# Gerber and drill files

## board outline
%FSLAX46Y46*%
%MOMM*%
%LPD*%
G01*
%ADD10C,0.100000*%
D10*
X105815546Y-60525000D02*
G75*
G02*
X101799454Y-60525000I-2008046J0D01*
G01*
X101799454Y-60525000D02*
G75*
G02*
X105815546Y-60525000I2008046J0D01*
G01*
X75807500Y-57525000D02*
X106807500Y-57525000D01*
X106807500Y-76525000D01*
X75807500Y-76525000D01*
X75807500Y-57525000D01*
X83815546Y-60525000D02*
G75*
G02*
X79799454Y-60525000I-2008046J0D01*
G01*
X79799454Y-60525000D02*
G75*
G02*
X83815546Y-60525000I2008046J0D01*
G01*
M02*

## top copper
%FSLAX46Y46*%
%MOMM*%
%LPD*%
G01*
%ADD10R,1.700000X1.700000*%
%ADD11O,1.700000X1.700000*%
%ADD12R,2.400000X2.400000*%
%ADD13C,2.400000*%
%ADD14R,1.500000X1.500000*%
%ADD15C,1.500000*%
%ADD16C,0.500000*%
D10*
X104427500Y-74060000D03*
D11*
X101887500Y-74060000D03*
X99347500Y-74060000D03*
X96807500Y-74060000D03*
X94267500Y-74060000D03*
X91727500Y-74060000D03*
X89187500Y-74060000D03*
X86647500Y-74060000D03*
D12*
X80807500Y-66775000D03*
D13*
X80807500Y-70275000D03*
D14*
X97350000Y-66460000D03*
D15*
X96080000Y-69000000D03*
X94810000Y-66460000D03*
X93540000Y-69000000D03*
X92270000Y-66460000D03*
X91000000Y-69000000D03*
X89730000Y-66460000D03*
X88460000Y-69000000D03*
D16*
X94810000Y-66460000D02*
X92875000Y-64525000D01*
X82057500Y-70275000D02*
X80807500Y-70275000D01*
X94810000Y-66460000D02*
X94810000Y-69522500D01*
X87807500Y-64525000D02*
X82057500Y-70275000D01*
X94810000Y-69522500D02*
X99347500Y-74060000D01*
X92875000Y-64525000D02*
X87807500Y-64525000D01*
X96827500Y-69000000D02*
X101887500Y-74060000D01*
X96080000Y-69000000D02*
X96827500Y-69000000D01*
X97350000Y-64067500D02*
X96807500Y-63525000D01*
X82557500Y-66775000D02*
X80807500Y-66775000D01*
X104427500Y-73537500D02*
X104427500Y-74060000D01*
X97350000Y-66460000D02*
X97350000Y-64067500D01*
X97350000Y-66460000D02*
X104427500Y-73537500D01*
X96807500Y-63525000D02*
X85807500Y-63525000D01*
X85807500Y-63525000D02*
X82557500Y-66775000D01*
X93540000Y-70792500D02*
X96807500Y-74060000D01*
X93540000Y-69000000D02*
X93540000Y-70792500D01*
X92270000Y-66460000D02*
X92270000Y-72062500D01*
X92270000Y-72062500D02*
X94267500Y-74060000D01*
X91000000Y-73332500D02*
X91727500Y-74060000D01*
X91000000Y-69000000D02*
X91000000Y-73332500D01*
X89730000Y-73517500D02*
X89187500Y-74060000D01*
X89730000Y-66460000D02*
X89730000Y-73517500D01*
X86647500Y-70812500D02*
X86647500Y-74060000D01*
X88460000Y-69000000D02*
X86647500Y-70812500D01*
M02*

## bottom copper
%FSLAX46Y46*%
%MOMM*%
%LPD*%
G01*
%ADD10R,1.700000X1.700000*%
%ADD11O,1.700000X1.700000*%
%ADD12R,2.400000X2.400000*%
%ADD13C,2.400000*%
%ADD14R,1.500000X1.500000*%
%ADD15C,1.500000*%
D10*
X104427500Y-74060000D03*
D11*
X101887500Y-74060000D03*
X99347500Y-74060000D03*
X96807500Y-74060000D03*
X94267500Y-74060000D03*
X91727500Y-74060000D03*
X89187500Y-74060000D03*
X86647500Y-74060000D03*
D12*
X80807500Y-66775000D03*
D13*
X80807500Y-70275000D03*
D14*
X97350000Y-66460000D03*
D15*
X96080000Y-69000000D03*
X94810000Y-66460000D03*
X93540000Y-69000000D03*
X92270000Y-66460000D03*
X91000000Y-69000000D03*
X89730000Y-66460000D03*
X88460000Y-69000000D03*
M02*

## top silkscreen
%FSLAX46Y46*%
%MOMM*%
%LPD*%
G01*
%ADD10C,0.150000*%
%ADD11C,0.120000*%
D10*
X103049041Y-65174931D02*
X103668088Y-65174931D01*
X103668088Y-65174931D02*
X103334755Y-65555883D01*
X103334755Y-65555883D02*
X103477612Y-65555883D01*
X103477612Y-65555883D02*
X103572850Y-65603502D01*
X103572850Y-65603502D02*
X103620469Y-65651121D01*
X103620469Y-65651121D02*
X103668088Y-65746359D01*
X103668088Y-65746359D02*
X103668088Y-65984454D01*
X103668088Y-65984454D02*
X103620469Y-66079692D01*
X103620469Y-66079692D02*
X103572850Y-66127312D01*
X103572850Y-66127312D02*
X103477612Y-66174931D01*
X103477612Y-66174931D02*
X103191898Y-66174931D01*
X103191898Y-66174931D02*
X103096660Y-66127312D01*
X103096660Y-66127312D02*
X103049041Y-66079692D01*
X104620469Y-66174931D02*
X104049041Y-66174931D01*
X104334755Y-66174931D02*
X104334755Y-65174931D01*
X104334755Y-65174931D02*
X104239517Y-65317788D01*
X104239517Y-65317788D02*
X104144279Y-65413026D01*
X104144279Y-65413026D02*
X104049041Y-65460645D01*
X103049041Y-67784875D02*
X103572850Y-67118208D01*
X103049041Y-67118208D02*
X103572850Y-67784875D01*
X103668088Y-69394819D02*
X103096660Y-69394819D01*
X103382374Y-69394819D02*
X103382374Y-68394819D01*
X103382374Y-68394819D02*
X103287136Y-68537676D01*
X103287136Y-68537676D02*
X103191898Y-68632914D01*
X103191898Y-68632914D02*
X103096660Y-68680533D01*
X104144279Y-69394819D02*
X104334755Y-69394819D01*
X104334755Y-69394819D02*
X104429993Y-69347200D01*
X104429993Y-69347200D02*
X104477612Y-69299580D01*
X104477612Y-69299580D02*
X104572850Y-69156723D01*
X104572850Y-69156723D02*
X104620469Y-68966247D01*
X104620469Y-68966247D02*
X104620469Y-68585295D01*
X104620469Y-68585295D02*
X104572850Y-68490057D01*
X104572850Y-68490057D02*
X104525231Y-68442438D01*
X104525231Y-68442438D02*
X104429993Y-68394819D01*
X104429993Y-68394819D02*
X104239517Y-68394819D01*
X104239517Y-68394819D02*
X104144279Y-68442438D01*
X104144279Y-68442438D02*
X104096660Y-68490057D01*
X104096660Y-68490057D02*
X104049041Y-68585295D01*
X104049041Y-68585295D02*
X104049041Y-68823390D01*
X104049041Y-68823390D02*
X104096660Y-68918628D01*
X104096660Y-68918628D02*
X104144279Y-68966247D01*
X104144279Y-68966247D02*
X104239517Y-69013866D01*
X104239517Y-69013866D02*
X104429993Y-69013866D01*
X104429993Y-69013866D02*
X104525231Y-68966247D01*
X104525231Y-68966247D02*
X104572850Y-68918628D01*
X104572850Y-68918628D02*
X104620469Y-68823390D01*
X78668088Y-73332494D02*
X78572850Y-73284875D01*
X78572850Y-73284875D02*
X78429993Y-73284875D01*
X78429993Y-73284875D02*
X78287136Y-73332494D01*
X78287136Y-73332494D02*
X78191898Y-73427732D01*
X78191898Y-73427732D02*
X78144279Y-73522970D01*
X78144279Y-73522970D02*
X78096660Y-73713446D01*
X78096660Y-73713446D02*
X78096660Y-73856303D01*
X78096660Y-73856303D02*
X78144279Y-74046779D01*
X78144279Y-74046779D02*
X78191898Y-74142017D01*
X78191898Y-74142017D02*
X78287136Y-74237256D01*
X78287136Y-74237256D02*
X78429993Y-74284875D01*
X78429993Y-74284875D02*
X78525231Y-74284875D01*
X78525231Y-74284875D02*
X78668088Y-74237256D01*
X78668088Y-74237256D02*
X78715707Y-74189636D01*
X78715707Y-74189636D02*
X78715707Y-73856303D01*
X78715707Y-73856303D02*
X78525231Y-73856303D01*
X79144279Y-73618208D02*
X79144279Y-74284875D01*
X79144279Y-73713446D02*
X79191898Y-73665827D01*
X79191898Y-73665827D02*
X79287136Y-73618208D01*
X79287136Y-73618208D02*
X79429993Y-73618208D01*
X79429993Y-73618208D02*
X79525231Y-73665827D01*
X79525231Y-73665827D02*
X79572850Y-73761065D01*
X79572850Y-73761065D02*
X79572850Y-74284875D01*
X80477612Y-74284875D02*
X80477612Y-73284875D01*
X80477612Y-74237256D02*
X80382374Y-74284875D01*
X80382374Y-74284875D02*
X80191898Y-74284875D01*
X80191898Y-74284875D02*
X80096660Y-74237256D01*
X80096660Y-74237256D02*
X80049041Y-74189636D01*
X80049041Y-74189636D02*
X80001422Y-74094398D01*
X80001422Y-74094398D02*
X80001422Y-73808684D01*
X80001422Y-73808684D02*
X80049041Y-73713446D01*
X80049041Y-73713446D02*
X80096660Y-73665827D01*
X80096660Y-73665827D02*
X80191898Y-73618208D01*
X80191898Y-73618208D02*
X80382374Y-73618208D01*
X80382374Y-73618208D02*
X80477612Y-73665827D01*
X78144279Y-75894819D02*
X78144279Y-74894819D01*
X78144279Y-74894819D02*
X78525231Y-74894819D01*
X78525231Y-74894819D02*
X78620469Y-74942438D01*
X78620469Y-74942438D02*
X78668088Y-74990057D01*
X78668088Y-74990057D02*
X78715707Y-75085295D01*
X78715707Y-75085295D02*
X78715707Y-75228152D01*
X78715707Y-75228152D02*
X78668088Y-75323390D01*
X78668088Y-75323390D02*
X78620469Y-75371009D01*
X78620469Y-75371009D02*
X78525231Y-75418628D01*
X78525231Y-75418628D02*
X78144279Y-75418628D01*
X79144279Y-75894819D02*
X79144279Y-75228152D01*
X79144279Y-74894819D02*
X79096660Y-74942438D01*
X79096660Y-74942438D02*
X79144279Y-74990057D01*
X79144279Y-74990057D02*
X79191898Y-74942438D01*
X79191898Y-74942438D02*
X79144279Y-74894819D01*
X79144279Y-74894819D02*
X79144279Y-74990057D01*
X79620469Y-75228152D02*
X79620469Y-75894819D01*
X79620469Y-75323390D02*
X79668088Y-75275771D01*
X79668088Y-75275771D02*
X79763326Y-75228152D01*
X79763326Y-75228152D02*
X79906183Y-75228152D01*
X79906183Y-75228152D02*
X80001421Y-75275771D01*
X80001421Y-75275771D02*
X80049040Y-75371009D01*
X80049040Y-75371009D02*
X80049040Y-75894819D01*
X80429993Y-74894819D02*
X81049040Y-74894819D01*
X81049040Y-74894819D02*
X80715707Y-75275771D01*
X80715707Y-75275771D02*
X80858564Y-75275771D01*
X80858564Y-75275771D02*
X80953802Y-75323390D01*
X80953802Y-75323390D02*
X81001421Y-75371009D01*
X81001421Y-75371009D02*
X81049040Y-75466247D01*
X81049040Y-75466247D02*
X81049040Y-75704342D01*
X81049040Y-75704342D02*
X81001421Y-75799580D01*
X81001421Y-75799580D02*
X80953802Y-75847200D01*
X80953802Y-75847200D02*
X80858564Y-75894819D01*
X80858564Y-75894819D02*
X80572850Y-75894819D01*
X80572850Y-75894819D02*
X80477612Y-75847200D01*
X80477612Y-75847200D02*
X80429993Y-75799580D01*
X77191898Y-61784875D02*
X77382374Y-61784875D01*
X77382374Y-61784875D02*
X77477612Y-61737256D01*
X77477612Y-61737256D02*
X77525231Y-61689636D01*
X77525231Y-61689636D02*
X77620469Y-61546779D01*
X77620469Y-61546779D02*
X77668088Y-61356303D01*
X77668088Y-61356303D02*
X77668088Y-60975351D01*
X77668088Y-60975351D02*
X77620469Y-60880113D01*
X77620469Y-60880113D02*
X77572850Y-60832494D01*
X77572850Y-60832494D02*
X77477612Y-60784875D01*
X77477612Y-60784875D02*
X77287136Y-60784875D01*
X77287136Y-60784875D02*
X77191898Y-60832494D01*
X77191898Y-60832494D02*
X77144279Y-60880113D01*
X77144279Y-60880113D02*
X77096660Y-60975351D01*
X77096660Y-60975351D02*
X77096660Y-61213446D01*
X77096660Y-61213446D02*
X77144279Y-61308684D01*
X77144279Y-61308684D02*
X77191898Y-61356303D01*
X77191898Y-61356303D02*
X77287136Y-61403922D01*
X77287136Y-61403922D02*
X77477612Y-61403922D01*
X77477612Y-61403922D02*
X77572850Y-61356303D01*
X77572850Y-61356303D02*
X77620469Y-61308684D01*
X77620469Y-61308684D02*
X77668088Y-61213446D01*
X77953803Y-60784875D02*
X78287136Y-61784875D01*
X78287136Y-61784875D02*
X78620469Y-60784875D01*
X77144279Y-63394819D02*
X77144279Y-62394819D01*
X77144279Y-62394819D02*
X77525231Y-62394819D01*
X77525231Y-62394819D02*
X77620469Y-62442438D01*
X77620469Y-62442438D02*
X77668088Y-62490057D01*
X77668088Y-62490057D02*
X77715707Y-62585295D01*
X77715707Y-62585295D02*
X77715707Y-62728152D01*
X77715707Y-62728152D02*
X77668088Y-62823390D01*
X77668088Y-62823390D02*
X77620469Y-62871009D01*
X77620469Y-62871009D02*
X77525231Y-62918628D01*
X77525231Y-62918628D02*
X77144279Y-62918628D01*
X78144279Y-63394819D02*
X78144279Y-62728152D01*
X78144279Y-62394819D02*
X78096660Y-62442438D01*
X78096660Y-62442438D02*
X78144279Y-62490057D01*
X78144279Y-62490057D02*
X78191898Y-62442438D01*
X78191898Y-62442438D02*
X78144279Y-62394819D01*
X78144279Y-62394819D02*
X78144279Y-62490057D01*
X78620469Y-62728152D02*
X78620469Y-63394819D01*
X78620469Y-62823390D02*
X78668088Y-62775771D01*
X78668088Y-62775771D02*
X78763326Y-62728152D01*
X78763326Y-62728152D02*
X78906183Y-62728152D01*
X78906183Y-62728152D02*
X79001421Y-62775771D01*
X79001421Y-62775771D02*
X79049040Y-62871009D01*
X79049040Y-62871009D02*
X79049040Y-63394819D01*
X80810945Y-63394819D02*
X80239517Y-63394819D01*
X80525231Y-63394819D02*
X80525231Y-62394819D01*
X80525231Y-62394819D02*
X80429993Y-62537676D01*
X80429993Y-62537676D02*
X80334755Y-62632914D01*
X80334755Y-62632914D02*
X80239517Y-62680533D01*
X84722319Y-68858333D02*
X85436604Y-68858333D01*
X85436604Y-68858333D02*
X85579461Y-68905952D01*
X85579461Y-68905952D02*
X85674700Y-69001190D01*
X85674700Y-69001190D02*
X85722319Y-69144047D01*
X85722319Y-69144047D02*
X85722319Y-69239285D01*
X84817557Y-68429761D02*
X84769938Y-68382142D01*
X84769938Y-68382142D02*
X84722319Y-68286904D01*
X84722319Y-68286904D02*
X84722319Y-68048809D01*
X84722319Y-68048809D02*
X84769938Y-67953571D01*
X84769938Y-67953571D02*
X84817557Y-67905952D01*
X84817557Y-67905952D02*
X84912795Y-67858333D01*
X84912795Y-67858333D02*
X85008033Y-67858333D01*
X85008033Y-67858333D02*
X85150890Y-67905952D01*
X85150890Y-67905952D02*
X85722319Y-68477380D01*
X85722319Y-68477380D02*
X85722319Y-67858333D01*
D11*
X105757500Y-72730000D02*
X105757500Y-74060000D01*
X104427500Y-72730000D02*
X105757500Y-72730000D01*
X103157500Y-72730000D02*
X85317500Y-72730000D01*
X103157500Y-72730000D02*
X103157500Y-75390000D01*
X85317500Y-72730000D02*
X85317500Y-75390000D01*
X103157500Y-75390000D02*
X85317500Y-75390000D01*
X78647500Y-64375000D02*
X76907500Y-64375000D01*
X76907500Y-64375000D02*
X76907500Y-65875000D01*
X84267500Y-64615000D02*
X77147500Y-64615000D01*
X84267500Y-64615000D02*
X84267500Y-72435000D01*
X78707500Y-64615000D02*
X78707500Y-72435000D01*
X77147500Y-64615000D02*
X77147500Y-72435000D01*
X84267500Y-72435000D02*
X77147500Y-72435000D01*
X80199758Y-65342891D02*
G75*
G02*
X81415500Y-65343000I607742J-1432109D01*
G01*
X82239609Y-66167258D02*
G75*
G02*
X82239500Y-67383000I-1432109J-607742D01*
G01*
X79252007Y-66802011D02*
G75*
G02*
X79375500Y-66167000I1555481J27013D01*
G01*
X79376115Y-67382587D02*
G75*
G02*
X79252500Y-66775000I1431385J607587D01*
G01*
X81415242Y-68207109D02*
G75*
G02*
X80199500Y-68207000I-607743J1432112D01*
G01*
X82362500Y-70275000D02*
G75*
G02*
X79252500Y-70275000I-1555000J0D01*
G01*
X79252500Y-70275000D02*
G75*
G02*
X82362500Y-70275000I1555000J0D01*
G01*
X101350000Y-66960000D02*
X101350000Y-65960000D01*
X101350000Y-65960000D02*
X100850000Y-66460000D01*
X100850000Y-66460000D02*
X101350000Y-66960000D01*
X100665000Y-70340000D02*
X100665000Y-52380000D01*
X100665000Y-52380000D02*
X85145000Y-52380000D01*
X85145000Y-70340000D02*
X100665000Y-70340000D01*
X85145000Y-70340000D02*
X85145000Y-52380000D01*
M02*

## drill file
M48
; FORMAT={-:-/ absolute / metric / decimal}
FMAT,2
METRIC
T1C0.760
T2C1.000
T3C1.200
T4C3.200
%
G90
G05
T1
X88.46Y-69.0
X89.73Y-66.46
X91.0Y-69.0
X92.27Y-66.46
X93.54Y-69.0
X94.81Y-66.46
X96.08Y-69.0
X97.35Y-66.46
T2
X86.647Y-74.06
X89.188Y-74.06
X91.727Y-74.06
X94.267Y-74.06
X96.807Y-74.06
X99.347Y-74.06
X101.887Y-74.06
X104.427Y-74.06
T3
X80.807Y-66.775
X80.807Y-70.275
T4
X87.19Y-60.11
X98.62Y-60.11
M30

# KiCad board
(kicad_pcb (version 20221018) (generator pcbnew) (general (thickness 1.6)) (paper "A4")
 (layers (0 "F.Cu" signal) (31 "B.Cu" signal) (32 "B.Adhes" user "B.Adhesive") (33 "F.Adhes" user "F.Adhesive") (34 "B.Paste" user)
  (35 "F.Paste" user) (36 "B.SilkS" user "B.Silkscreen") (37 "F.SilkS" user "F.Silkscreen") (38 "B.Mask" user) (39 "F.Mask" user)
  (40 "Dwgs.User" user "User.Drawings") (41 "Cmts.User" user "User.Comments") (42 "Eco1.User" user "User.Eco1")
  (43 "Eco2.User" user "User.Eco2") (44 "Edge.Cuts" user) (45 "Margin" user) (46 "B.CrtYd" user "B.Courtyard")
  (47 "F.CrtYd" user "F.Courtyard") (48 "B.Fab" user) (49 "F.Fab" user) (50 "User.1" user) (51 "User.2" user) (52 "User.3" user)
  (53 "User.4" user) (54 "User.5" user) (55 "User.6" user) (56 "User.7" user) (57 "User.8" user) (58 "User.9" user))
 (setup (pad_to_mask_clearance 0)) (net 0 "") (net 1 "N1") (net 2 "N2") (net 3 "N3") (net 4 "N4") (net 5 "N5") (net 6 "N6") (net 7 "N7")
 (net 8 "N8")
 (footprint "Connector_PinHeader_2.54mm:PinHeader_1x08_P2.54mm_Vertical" (layer "F.Cu") (at 104.4275 74.06 -90)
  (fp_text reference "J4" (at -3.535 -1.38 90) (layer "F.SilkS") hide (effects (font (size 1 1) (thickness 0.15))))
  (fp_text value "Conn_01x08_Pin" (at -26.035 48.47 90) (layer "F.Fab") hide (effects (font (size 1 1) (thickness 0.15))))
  (fp_line (start -1.33 -1.33) (end 0 -1.33) (stroke (width 0.12) (type solid)) (layer "F.SilkS"))
  (fp_line (start -1.33 0) (end -1.33 -1.33) (stroke (width 0.12) (type solid)) (layer "F.SilkS"))
  (fp_line (start -1.33 1.27) (end -1.33 19.11) (stroke (width 0.12) (type solid)) (layer "F.SilkS"))
  (fp_line (start -1.33 1.27) (end 1.33 1.27) (stroke (width 0.12) (type solid)) (layer "F.SilkS"))
  (fp_line (start -1.33 19.11) (end 1.33 19.11) (stroke (width 0.12) (type solid)) (layer "F.SilkS"))
  (fp_line (start 1.33 1.27) (end 1.33 19.11) (stroke (width 0.12) (type solid)) (layer "F.SilkS"))
  (pad "1" thru_hole rect (at 0 0 270) (size 1.7 1.7) (drill 1) (layers "*.Cu" "*.Mask") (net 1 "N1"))
  (pad "2" thru_hole oval (at 0 2.54 270) (size 1.7 1.7) (drill 1) (layers "*.Cu" "*.Mask") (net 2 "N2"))
  (pad "3" thru_hole oval (at 0 5.08 270) (size 1.7 1.7) (drill 1) (layers "*.Cu" "*.Mask") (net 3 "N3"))
  (pad "4" thru_hole oval (at 0 7.62 270) (size 1.7 1.7) (drill 1) (layers "*.Cu" "*.Mask") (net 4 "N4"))
  (pad "5" thru_hole oval (at 0 10.16 270) (size 1.7 1.7) (drill 1) (layers "*.Cu" "*.Mask") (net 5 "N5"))
  (pad "6" thru_hole oval (at 0 12.7 270) (size 1.7 1.7) (drill 1) (layers "*.Cu" "*.Mask") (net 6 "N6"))
  (pad "7" thru_hole oval (at 0 15.24 270) (size 1.7 1.7) (drill 1) (layers "*.Cu" "*.Mask") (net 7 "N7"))
  (pad "8" thru_hole oval (at 0 17.78 270) (size 1.7 1.7) (drill 1) (layers "*.Cu" "*.Mask") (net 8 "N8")))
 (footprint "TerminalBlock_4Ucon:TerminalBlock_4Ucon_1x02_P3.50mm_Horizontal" (layer "F.Cu") (at 80.8075 66.775 -90)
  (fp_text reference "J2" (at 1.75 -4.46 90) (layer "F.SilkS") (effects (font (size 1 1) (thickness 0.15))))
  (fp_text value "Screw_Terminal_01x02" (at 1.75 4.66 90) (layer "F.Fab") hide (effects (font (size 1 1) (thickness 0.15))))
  (fp_line (start -2.4 2.16) (end -2.4 3.9) (stroke (width 0.12) (type solid)) (layer "F.SilkS"))
  (fp_line (start -2.4 3.9) (end -0.9 3.9) (stroke (width 0.12) (type solid)) (layer "F.SilkS"))
  (fp_line (start -2.16 -3.46) (end -2.16 3.66) (stroke (width 0.12) (type solid)) (layer "F.SilkS"))
  (fp_line (start -2.16 -3.46) (end 5.66 -3.46) (stroke (width 0.12) (type solid)) (layer "F.SilkS"))
  (fp_line (start -2.16 2.1) (end 5.66 2.1) (stroke (width 0.12) (type solid)) (layer "F.SilkS"))
  (fp_line (start -2.16 3.66) (end 5.66 3.66) (stroke (width 0.12) (type solid)) (layer "F.SilkS"))
  (fp_line (start 5.66 -3.46) (end 5.66 3.66) (stroke (width 0.12) (type solid)) (layer "F.SilkS"))
  (fp_arc (start -1.432109 0.607742) (mid -1.555727 -0.00014) (end -1.432 -0.608) (stroke (width 0.12) (type solid)) (layer "F.SilkS"))
  (fp_arc (start -0.607742 -1.432109) (mid 0.00014 -1.555727) (end 0.608 -1.432) (stroke (width 0.12) (type solid)) (layer "F.SilkS"))
  (fp_arc (start 0.027011 1.555493) (mid -0.296984 1.527118) (end -0.608 1.432) (stroke (width 0.12) (type solid)) (layer "F.SilkS"))
  (fp_arc (start 0.607587 1.431385) (mid 0.310017 1.523783) (end 0 1.555) (stroke (width 0.12) (type solid)) (layer "F.SilkS"))
  (fp_arc (start 1.432109 -0.607742) (mid 1.555727 0.00014) (end 1.432 0.608) (stroke (width 0.12) (type solid)) (layer "F.SilkS"))
  (fp_circle (center 3.5 0) (end 5.055 0) (stroke (width 0.12) (type solid)) (fill none) (layer "F.SilkS"))
  (pad "1" thru_hole rect (at 0 0 270) (size 2.4 2.4) (drill 1.2) (layers "*.Cu" "*.Mask") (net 1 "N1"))
  (pad "2" thru_hole circle (at 3.5 0 270) (size 2.4 2.4) (drill 1.2) (layers "*.Cu" "*.Mask") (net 3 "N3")))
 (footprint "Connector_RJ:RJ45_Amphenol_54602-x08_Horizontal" (layer "F.Cu") (at 97.35 66.46 180)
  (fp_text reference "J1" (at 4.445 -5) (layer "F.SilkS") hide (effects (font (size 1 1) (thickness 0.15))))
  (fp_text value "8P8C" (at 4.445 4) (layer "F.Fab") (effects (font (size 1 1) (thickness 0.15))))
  (fp_line (start -4 -0.5) (end -4 0.5) (stroke (width 0.12) (type solid)) (layer "F.SilkS"))
  (fp_line (start -4 0.5) (end -3.5 0) (stroke (width 0.12) (type solid)) (layer "F.SilkS"))
  (fp_line (start -3.5 0) (end -4 -0.5) (stroke (width 0.12) (type solid)) (layer "F.SilkS"))
  (fp_line (start -3.315 -3.88) (end -3.315 14.08) (stroke (width 0.12) (type solid)) (layer "F.SilkS"))
  (fp_line (start -3.315 14.08) (end 12.205 14.08) (stroke (width 0.12) (type solid)) (layer "F.SilkS"))
  (fp_line (start 12.205 -3.88) (end -3.315 -3.88) (stroke (width 0.12) (type solid)) (layer "F.SilkS"))
  (fp_line (start 12.205 -3.88) (end 12.205 14.08) (stroke (width 0.12) (type solid)) (layer "F.SilkS"))
  (pad "" np_thru_hole circle (at -1.27 6.35 180) (size 3.2 3.2) (drill 3.2) (layers "*.Cu" "*.Mask"))
  (pad "" np_thru_hole circle (at 10.16 6.35 180) (size 3.2 3.2) (drill 3.2) (layers "*.Cu" "*.Mask"))
  (pad "1" thru_hole rect (at 0 0 180) (size 1.5 1.5) (drill 0.76) (layers "*.Cu" "*.Mask") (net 1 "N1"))
  (pad "2" thru_hole circle (at 1.27 -2.54 180) (size 1.5 1.5) (drill 0.76) (layers "*.Cu" "*.Mask") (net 2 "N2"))
  (pad "3" thru_hole circle (at 2.54 0 180) (size 1.5 1.5) (drill 0.76) (layers "*.Cu" "*.Mask") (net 3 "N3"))
  (pad "4" thru_hole circle (at 3.81 -2.54 180) (size 1.5 1.5) (drill 0.76) (layers "*.Cu" "*.Mask") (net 4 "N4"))
  (pad "5" thru_hole circle (at 5.08 0 180) (size 1.5 1.5) (drill 0.76) (layers "*.Cu" "*.Mask") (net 5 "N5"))
  (pad "6" thru_hole circle (at 6.35 -2.54 180) (size 1.5 1.5) (drill 0.76) (layers "*.Cu" "*.Mask") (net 6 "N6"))
  (pad "7" thru_hole circle (at 7.62 0 180) (size 1.5 1.5) (drill 0.76) (layers "*.Cu" "*.Mask") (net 7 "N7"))
  (pad "8" thru_hole circle (at 8.89 -2.54 180) (size 1.5 1.5) (drill 0.76) (layers "*.Cu" "*.Mask") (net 8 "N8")))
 (gr_circle (center 103.8075 60.525) (end 103.1725 62.43) (stroke (width 0.1) (type default)) (fill none) (layer "Edge.Cuts"))
 (gr_rect (start 75.8075 57.525) (end 106.8075 76.525) (stroke (width 0.1) (type default)) (fill none) (layer "Edge.Cuts"))
 (gr_circle (center 81.8075 60.525) (end 81.1725 62.43) (stroke (width 0.1) (type default)) (fill none) (layer "Edge.Cuts"))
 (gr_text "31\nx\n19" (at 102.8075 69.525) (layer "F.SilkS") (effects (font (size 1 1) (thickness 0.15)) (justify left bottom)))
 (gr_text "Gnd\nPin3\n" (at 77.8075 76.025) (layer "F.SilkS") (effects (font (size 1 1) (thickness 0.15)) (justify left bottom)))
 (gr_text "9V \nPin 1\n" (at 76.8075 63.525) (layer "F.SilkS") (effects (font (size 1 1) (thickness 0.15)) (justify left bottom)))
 (segment (start 94.81 66.46) (end 92.875 64.525) (width 0.5) (layer "F.Cu") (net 3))
 (segment (start 82.0575 70.275) (end 80.8075 70.275) (width 0.5) (layer "F.Cu") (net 3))
 (segment (start 94.81 66.46) (end 94.81 69.5225) (width 0.5) (layer "F.Cu") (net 3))
 (segment (start 87.8075 64.525) (end 82.0575 70.275) (width 0.5) (layer "F.Cu") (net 3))
 (segment (start 94.81 69.5225) (end 99.3475 74.06) (width 0.5) (layer "F.Cu") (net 3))
 (segment (start 92.875 64.525) (end 87.8075 64.525) (width 0.5) (layer "F.Cu") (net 3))
 (segment (start 96.8275 69) (end 101.8875 74.06) (width 0.5) (layer "F.Cu") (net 2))
 (segment (start 96.08 69) (end 96.8275 69) (width 0.5) (layer "F.Cu") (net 2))
 (segment (start 97.35 64.0675) (end 96.8075 63.525) (width 0.5) (layer "F.Cu") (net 1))
 (segment (start 82.5575 66.775) (end 80.8075 66.775) (width 0.5) (layer "F.Cu") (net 1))
 (segment (start 104.4275 73.5375) (end 104.4275 74.06) (width 0.5) (layer "F.Cu") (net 1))
 (segment (start 97.35 66.46) (end 97.35 64.0675) (width 0.5) (layer "F.Cu") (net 1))
 (segment (start 97.35 66.46) (end 104.4275 73.5375) (width 0.5) (layer "F.Cu") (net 1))
 (segment (start 96.8075 63.525) (end 85.8075 63.525) (width 0.5) (layer "F.Cu") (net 1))
 (segment (start 85.8075 63.525) (end 82.5575 66.775) (width 0.5) (layer "F.Cu") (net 1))
 (segment (start 93.54 70.7925) (end 96.8075 74.06) (width 0.5) (layer "F.Cu") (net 4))
 (segment (start 93.54 69) (end 93.54 70.7925) (width 0.5) (layer "F.Cu") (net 4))
 (segment (start 92.27 66.46) (end 92.27 72.0625) (width 0.5) (layer "F.Cu") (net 5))
 (segment (start 92.27 72.0625) (end 94.2675 74.06) (width 0.5) (layer "F.Cu") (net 5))
 (segment (start 91 73.3325) (end 91.7275 74.06) (width 0.5) (layer "F.Cu") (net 6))
 (segment (start 91 69) (end 91 73.3325) (width 0.5) (layer "F.Cu") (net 6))
 (segment (start 89.73 73.5175) (end 89.1875 74.06) (width 0.5) (layer "F.Cu") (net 7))
 (segment (start 89.73 66.46) (end 89.73 73.5175) (width 0.5) (layer "F.Cu") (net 7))
 (segment (start 86.6475 70.8125) (end 86.6475 74.06) (width 0.5) (layer "F.Cu") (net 8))
 (segment (start 88.46 69) (end 86.6475 70.8125) (width 0.5) (layer "F.Cu") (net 8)))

